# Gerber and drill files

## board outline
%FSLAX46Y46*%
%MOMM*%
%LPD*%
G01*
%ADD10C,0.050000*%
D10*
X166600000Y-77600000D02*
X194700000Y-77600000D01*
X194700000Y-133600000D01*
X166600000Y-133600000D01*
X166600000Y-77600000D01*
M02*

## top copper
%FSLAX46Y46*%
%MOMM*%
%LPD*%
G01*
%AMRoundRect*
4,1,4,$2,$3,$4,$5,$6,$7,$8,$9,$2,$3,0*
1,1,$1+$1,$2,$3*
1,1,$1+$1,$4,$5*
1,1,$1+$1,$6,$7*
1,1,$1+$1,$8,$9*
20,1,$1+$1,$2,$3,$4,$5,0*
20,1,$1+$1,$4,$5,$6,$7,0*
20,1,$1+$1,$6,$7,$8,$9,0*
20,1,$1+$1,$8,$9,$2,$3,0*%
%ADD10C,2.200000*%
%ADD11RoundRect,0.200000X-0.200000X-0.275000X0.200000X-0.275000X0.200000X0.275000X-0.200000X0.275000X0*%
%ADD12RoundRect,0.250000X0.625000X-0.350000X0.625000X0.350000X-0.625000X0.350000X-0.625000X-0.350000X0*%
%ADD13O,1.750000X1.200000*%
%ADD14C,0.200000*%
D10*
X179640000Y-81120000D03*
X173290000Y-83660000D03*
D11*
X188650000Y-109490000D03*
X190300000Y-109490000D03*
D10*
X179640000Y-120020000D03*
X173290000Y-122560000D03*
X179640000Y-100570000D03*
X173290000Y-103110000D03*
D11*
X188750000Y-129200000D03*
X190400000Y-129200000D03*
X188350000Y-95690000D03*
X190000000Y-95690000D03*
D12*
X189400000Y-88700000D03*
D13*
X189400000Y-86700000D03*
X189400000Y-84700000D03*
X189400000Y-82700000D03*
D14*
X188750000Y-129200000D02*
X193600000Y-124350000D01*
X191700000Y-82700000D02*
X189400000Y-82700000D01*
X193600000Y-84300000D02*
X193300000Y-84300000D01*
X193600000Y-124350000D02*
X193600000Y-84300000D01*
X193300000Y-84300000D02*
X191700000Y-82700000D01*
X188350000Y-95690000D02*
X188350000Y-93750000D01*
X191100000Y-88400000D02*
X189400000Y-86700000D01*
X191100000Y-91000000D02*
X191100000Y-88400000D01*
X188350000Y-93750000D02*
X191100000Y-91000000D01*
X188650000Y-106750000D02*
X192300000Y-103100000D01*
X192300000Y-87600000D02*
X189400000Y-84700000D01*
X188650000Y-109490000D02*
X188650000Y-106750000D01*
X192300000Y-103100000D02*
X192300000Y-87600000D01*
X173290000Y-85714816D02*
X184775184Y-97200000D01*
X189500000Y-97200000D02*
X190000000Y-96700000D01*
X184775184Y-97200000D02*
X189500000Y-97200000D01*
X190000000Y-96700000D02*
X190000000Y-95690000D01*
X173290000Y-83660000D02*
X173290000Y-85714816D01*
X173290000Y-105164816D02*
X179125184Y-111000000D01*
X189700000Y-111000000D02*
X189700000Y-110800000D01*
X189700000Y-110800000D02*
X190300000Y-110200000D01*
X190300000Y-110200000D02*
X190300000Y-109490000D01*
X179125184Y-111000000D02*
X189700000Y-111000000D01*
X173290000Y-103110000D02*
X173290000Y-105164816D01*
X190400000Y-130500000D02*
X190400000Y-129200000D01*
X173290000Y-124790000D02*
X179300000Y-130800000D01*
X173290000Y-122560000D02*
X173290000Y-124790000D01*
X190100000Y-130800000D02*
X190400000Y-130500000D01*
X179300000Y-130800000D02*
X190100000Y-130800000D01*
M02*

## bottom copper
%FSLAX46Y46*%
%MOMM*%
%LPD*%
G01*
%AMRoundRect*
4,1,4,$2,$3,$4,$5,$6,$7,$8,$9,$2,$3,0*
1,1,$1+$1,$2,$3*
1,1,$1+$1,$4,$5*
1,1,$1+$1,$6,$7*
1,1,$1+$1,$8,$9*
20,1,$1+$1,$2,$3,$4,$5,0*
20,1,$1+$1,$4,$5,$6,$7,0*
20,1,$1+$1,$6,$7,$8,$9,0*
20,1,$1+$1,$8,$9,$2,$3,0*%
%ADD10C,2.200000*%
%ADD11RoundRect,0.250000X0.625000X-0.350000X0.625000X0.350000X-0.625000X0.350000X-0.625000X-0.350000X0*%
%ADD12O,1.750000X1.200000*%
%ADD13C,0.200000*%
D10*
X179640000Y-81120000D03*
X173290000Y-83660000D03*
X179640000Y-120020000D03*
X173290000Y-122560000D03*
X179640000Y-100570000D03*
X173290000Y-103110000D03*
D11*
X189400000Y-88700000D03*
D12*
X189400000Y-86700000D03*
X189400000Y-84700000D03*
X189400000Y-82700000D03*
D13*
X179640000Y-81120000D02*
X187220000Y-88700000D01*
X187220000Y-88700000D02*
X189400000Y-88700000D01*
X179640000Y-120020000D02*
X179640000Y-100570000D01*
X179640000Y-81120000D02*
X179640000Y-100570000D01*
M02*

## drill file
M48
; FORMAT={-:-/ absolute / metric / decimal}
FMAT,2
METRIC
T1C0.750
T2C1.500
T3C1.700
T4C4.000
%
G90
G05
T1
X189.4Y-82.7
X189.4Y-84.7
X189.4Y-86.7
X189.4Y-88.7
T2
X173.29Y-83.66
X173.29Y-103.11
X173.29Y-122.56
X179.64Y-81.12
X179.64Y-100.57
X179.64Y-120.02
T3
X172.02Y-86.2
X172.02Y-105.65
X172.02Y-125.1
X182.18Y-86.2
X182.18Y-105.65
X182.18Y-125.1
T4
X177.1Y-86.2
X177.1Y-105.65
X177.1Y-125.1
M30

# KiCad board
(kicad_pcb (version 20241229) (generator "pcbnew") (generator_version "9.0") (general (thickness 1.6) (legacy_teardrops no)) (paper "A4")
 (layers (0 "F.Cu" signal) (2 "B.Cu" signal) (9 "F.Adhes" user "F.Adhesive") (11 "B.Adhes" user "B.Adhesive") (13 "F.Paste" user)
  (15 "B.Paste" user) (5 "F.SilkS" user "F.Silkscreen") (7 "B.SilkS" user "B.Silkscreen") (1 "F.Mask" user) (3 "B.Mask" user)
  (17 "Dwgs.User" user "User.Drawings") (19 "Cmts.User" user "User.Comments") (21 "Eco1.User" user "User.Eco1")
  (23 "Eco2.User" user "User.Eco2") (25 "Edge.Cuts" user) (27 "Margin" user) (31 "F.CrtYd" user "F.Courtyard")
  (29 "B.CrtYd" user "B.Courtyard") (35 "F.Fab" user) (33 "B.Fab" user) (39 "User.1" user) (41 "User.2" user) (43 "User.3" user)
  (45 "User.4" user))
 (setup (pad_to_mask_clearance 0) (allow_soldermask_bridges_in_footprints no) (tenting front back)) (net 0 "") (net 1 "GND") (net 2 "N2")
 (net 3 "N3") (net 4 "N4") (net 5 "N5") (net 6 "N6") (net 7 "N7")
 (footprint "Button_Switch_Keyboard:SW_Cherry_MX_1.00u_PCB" (layer "F.Cu") (at 179.64 81.12)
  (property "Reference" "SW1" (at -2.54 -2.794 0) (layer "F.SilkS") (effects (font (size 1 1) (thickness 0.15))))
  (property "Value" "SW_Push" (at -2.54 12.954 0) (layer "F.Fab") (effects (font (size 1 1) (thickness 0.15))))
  (pad "" np_thru_hole circle (at -7.62 5.08) (size 1.7 1.7) (drill 1.7) (layers "*.Cu" "*.Mask"))
  (pad "" np_thru_hole circle (at -2.54 5.08) (size 4 4) (drill 4) (layers "*.Cu" "*.Mask"))
  (pad "" np_thru_hole circle (at 2.54 5.08) (size 1.7 1.7) (drill 1.7) (layers "*.Cu" "*.Mask"))
  (pad "1" thru_hole circle (at 0 0) (size 2.2 2.2) (drill 1.5) (layers "*.Cu" "*.Mask") (remove_unused_layers no) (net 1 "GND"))
  (pad "2" thru_hole circle (at -6.35 2.54) (size 2.2 2.2) (drill 1.5) (layers "*.Cu" "*.Mask") (remove_unused_layers no) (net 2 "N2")))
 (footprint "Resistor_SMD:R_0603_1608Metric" (layer "F.Cu") (at 189.475 109.49)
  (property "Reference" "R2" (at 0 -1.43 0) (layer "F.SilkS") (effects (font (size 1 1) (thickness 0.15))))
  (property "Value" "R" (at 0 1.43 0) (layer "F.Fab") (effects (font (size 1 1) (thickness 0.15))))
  (pad "1" smd roundrect (at -0.825 0) (size 0.8 0.95) (layers "F.Cu" "F.Mask" "F.Paste") (roundrect_rratio 0.25) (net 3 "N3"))
  (pad "2" smd roundrect (at 0.825 0) (size 0.8 0.95) (layers "F.Cu" "F.Mask" "F.Paste") (roundrect_rratio 0.25) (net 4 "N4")))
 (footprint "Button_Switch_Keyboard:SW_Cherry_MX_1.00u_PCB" (layer "F.Cu") (at 179.64 120.02)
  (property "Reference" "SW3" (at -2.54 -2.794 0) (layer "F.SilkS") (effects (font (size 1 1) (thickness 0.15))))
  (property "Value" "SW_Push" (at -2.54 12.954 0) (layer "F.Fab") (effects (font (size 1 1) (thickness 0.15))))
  (pad "" np_thru_hole circle (at -7.62 5.08) (size 1.7 1.7) (drill 1.7) (layers "*.Cu" "*.Mask"))
  (pad "" np_thru_hole circle (at -2.54 5.08) (size 4 4) (drill 4) (layers "*.Cu" "*.Mask"))
  (pad "" np_thru_hole circle (at 2.54 5.08) (size 1.7 1.7) (drill 1.7) (layers "*.Cu" "*.Mask"))
  (pad "1" thru_hole circle (at 0 0) (size 2.2 2.2) (drill 1.5) (layers "*.Cu" "*.Mask") (remove_unused_layers no) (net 1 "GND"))
  (pad "2" thru_hole circle (at -6.35 2.54) (size 2.2 2.2) (drill 1.5) (layers "*.Cu" "*.Mask") (remove_unused_layers no) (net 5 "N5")))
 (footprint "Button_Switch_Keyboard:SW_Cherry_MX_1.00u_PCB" (layer "F.Cu") (at 179.64 100.57)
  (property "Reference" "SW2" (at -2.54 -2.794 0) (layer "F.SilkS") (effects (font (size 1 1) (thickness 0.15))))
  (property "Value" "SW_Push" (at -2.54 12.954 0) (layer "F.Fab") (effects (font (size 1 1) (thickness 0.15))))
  (pad "" np_thru_hole circle (at -7.62 5.08) (size 1.7 1.7) (drill 1.7) (layers "*.Cu" "*.Mask"))
  (pad "" np_thru_hole circle (at -2.54 5.08) (size 4 4) (drill 4) (layers "*.Cu" "*.Mask"))
  (pad "" np_thru_hole circle (at 2.54 5.08) (size 1.7 1.7) (drill 1.7) (layers "*.Cu" "*.Mask"))
  (pad "1" thru_hole circle (at 0 0) (size 2.2 2.2) (drill 1.5) (layers "*.Cu" "*.Mask") (remove_unused_layers no) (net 1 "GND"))
  (pad "2" thru_hole circle (at -6.35 2.54) (size 2.2 2.2) (drill 1.5) (layers "*.Cu" "*.Mask") (remove_unused_layers no) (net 4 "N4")))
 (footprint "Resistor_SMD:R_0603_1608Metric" (layer "F.Cu") (at 189.575 129.2)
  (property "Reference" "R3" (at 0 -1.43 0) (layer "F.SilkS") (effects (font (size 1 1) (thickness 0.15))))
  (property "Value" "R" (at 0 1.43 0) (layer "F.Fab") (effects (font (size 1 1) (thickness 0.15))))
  (pad "1" smd roundrect (at -0.825 0) (size 0.8 0.95) (layers "F.Cu" "F.Mask" "F.Paste") (roundrect_rratio 0.25) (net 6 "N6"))
  (pad "2" smd roundrect (at 0.825 0) (size 0.8 0.95) (layers "F.Cu" "F.Mask" "F.Paste") (roundrect_rratio 0.25) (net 5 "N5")))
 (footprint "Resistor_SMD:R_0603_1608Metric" (layer "F.Cu") (at 189.175 95.69)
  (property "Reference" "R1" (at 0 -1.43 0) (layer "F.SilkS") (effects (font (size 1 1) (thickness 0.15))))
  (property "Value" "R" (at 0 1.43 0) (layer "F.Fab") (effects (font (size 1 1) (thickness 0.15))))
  (pad "1" smd roundrect (at -0.825 0) (size 0.8 0.95) (layers "F.Cu" "F.Mask" "F.Paste") (roundrect_rratio 0.25) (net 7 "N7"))
  (pad "2" smd roundrect (at 0.825 0) (size 0.8 0.95) (layers "F.Cu" "F.Mask" "F.Paste") (roundrect_rratio 0.25) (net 2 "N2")))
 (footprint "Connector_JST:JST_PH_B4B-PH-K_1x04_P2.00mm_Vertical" (layer "F.Cu") (at 189.4 88.7 90)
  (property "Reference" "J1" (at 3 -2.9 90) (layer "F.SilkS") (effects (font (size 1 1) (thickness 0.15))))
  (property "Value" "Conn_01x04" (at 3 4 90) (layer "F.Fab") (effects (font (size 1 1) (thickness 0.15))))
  (pad "1" thru_hole roundrect (at 0 0 90) (size 1.2 1.75) (drill 0.75) (layers "*.Cu" "*.Mask") (remove_unused_layers no)
   (roundrect_rratio 0.208333) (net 1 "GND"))
  (pad "2" thru_hole oval (at 2 0 90) (size 1.2 1.75) (drill 0.75) (layers "*.Cu" "*.Mask") (remove_unused_layers no) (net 7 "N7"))
  (pad "3" thru_hole oval (at 4 0 90) (size 1.2 1.75) (drill 0.75) (layers "*.Cu" "*.Mask") (remove_unused_layers no) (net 3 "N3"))
  (pad "4" thru_hole oval (at 6 0 90) (size 1.2 1.75) (drill 0.75) (layers "*.Cu" "*.Mask") (remove_unused_layers no) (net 6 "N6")))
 (gr_rect (start 166.6 77.6) (end 194.7 133.6) (stroke (width 0.05) (type default)) (fill no) (layer "Edge.Cuts"))
 (segment (start 188.75 129.2) (end 193.6 124.35) (width 0.2) (layer "F.Cu") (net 6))
 (segment (start 191.7 82.7) (end 189.4 82.7) (width 0.2) (layer "F.Cu") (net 6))
 (segment (start 193.6 84.3) (end 193.3 84.3) (width 0.2) (layer "F.Cu") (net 6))
 (segment (start 193.6 124.35) (end 193.6 84.3) (width 0.2) (layer "F.Cu") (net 6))
 (segment (start 193.3 84.3) (end 191.7 82.7) (width 0.2) (layer "F.Cu") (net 6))
 (segment (start 179.64 81.12) (end 187.22 88.7) (width 0.2) (layer "B.Cu") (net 1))
 (segment (start 187.22 88.7) (end 189.4 88.7) (width 0.2) (layer "B.Cu") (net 1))
 (segment (start 179.64 120.02) (end 179.64 100.57) (width 0.2) (layer "B.Cu") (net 1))
 (segment (start 179.64 81.12) (end 179.64 100.57) (width 0.2) (layer "B.Cu") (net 1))
 (segment (start 188.35 95.69) (end 188.35 93.75) (width 0.2) (layer "F.Cu") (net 7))
 (segment (start 191.1 88.4) (end 189.4 86.7) (width 0.2) (layer "F.Cu") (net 7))
 (segment (start 191.1 91) (end 191.1 88.4) (width 0.2) (layer "F.Cu") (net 7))
 (segment (start 188.35 93.75) (end 191.1 91) (width 0.2) (layer "F.Cu") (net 7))
 (segment (start 188.65 106.75) (end 192.3 103.1) (width 0.2) (layer "F.Cu") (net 3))
 (segment (start 192.3 87.6) (end 189.4 84.7) (width 0.2) (layer "F.Cu") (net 3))
 (segment (start 188.65 109.49) (end 188.65 106.75) (width 0.2) (layer "F.Cu") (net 3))
 (segment (start 192.3 103.1) (end 192.3 87.6) (width 0.2) (layer "F.Cu") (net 3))
 (segment (start 173.29 85.714816) (end 184.775184 97.2) (width 0.2) (layer "F.Cu") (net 2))
 (segment (start 189.5 97.2) (end 190 96.7) (width 0.2) (layer "F.Cu") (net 2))
 (segment (start 184.775184 97.2) (end 189.5 97.2) (width 0.2) (layer "F.Cu") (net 2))
 (segment (start 190 96.7) (end 190 95.69) (width 0.2) (layer "F.Cu") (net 2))
 (segment (start 173.29 83.66) (end 173.29 85.714816) (width 0.2) (layer "F.Cu") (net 2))
 (segment (start 173.29 105.164816) (end 179.125184 111) (width 0.2) (layer "F.Cu") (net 4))
 (segment (start 189.7 111) (end 189.7 110.8) (width 0.2) (layer "F.Cu") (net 4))
 (segment (start 189.7 110.8) (end 190.3 110.2) (width 0.2) (layer "F.Cu") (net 4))
 (segment (start 190.3 110.2) (end 190.3 109.49) (width 0.2) (layer "F.Cu") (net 4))
 (segment (start 179.125184 111) (end 189.7 111) (width 0.2) (layer "F.Cu") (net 4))
 (segment (start 173.29 103.11) (end 173.29 105.164816) (width 0.2) (layer "F.Cu") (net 4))
 (segment (start 190.4 130.5) (end 190.4 129.2) (width 0.2) (layer "F.Cu") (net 5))
 (segment (start 173.29 124.79) (end 179.3 130.8) (width 0.2) (layer "F.Cu") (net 5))
 (segment (start 173.29 122.56) (end 173.29 124.79) (width 0.2) (layer "F.Cu") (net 5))
 (segment (start 190.1 130.8) (end 190.4 130.5) (width 0.2) (layer "F.Cu") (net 5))
 (segment (start 179.3 130.8) (end 190.1 130.8) (width 0.2) (layer "F.Cu") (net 5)))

